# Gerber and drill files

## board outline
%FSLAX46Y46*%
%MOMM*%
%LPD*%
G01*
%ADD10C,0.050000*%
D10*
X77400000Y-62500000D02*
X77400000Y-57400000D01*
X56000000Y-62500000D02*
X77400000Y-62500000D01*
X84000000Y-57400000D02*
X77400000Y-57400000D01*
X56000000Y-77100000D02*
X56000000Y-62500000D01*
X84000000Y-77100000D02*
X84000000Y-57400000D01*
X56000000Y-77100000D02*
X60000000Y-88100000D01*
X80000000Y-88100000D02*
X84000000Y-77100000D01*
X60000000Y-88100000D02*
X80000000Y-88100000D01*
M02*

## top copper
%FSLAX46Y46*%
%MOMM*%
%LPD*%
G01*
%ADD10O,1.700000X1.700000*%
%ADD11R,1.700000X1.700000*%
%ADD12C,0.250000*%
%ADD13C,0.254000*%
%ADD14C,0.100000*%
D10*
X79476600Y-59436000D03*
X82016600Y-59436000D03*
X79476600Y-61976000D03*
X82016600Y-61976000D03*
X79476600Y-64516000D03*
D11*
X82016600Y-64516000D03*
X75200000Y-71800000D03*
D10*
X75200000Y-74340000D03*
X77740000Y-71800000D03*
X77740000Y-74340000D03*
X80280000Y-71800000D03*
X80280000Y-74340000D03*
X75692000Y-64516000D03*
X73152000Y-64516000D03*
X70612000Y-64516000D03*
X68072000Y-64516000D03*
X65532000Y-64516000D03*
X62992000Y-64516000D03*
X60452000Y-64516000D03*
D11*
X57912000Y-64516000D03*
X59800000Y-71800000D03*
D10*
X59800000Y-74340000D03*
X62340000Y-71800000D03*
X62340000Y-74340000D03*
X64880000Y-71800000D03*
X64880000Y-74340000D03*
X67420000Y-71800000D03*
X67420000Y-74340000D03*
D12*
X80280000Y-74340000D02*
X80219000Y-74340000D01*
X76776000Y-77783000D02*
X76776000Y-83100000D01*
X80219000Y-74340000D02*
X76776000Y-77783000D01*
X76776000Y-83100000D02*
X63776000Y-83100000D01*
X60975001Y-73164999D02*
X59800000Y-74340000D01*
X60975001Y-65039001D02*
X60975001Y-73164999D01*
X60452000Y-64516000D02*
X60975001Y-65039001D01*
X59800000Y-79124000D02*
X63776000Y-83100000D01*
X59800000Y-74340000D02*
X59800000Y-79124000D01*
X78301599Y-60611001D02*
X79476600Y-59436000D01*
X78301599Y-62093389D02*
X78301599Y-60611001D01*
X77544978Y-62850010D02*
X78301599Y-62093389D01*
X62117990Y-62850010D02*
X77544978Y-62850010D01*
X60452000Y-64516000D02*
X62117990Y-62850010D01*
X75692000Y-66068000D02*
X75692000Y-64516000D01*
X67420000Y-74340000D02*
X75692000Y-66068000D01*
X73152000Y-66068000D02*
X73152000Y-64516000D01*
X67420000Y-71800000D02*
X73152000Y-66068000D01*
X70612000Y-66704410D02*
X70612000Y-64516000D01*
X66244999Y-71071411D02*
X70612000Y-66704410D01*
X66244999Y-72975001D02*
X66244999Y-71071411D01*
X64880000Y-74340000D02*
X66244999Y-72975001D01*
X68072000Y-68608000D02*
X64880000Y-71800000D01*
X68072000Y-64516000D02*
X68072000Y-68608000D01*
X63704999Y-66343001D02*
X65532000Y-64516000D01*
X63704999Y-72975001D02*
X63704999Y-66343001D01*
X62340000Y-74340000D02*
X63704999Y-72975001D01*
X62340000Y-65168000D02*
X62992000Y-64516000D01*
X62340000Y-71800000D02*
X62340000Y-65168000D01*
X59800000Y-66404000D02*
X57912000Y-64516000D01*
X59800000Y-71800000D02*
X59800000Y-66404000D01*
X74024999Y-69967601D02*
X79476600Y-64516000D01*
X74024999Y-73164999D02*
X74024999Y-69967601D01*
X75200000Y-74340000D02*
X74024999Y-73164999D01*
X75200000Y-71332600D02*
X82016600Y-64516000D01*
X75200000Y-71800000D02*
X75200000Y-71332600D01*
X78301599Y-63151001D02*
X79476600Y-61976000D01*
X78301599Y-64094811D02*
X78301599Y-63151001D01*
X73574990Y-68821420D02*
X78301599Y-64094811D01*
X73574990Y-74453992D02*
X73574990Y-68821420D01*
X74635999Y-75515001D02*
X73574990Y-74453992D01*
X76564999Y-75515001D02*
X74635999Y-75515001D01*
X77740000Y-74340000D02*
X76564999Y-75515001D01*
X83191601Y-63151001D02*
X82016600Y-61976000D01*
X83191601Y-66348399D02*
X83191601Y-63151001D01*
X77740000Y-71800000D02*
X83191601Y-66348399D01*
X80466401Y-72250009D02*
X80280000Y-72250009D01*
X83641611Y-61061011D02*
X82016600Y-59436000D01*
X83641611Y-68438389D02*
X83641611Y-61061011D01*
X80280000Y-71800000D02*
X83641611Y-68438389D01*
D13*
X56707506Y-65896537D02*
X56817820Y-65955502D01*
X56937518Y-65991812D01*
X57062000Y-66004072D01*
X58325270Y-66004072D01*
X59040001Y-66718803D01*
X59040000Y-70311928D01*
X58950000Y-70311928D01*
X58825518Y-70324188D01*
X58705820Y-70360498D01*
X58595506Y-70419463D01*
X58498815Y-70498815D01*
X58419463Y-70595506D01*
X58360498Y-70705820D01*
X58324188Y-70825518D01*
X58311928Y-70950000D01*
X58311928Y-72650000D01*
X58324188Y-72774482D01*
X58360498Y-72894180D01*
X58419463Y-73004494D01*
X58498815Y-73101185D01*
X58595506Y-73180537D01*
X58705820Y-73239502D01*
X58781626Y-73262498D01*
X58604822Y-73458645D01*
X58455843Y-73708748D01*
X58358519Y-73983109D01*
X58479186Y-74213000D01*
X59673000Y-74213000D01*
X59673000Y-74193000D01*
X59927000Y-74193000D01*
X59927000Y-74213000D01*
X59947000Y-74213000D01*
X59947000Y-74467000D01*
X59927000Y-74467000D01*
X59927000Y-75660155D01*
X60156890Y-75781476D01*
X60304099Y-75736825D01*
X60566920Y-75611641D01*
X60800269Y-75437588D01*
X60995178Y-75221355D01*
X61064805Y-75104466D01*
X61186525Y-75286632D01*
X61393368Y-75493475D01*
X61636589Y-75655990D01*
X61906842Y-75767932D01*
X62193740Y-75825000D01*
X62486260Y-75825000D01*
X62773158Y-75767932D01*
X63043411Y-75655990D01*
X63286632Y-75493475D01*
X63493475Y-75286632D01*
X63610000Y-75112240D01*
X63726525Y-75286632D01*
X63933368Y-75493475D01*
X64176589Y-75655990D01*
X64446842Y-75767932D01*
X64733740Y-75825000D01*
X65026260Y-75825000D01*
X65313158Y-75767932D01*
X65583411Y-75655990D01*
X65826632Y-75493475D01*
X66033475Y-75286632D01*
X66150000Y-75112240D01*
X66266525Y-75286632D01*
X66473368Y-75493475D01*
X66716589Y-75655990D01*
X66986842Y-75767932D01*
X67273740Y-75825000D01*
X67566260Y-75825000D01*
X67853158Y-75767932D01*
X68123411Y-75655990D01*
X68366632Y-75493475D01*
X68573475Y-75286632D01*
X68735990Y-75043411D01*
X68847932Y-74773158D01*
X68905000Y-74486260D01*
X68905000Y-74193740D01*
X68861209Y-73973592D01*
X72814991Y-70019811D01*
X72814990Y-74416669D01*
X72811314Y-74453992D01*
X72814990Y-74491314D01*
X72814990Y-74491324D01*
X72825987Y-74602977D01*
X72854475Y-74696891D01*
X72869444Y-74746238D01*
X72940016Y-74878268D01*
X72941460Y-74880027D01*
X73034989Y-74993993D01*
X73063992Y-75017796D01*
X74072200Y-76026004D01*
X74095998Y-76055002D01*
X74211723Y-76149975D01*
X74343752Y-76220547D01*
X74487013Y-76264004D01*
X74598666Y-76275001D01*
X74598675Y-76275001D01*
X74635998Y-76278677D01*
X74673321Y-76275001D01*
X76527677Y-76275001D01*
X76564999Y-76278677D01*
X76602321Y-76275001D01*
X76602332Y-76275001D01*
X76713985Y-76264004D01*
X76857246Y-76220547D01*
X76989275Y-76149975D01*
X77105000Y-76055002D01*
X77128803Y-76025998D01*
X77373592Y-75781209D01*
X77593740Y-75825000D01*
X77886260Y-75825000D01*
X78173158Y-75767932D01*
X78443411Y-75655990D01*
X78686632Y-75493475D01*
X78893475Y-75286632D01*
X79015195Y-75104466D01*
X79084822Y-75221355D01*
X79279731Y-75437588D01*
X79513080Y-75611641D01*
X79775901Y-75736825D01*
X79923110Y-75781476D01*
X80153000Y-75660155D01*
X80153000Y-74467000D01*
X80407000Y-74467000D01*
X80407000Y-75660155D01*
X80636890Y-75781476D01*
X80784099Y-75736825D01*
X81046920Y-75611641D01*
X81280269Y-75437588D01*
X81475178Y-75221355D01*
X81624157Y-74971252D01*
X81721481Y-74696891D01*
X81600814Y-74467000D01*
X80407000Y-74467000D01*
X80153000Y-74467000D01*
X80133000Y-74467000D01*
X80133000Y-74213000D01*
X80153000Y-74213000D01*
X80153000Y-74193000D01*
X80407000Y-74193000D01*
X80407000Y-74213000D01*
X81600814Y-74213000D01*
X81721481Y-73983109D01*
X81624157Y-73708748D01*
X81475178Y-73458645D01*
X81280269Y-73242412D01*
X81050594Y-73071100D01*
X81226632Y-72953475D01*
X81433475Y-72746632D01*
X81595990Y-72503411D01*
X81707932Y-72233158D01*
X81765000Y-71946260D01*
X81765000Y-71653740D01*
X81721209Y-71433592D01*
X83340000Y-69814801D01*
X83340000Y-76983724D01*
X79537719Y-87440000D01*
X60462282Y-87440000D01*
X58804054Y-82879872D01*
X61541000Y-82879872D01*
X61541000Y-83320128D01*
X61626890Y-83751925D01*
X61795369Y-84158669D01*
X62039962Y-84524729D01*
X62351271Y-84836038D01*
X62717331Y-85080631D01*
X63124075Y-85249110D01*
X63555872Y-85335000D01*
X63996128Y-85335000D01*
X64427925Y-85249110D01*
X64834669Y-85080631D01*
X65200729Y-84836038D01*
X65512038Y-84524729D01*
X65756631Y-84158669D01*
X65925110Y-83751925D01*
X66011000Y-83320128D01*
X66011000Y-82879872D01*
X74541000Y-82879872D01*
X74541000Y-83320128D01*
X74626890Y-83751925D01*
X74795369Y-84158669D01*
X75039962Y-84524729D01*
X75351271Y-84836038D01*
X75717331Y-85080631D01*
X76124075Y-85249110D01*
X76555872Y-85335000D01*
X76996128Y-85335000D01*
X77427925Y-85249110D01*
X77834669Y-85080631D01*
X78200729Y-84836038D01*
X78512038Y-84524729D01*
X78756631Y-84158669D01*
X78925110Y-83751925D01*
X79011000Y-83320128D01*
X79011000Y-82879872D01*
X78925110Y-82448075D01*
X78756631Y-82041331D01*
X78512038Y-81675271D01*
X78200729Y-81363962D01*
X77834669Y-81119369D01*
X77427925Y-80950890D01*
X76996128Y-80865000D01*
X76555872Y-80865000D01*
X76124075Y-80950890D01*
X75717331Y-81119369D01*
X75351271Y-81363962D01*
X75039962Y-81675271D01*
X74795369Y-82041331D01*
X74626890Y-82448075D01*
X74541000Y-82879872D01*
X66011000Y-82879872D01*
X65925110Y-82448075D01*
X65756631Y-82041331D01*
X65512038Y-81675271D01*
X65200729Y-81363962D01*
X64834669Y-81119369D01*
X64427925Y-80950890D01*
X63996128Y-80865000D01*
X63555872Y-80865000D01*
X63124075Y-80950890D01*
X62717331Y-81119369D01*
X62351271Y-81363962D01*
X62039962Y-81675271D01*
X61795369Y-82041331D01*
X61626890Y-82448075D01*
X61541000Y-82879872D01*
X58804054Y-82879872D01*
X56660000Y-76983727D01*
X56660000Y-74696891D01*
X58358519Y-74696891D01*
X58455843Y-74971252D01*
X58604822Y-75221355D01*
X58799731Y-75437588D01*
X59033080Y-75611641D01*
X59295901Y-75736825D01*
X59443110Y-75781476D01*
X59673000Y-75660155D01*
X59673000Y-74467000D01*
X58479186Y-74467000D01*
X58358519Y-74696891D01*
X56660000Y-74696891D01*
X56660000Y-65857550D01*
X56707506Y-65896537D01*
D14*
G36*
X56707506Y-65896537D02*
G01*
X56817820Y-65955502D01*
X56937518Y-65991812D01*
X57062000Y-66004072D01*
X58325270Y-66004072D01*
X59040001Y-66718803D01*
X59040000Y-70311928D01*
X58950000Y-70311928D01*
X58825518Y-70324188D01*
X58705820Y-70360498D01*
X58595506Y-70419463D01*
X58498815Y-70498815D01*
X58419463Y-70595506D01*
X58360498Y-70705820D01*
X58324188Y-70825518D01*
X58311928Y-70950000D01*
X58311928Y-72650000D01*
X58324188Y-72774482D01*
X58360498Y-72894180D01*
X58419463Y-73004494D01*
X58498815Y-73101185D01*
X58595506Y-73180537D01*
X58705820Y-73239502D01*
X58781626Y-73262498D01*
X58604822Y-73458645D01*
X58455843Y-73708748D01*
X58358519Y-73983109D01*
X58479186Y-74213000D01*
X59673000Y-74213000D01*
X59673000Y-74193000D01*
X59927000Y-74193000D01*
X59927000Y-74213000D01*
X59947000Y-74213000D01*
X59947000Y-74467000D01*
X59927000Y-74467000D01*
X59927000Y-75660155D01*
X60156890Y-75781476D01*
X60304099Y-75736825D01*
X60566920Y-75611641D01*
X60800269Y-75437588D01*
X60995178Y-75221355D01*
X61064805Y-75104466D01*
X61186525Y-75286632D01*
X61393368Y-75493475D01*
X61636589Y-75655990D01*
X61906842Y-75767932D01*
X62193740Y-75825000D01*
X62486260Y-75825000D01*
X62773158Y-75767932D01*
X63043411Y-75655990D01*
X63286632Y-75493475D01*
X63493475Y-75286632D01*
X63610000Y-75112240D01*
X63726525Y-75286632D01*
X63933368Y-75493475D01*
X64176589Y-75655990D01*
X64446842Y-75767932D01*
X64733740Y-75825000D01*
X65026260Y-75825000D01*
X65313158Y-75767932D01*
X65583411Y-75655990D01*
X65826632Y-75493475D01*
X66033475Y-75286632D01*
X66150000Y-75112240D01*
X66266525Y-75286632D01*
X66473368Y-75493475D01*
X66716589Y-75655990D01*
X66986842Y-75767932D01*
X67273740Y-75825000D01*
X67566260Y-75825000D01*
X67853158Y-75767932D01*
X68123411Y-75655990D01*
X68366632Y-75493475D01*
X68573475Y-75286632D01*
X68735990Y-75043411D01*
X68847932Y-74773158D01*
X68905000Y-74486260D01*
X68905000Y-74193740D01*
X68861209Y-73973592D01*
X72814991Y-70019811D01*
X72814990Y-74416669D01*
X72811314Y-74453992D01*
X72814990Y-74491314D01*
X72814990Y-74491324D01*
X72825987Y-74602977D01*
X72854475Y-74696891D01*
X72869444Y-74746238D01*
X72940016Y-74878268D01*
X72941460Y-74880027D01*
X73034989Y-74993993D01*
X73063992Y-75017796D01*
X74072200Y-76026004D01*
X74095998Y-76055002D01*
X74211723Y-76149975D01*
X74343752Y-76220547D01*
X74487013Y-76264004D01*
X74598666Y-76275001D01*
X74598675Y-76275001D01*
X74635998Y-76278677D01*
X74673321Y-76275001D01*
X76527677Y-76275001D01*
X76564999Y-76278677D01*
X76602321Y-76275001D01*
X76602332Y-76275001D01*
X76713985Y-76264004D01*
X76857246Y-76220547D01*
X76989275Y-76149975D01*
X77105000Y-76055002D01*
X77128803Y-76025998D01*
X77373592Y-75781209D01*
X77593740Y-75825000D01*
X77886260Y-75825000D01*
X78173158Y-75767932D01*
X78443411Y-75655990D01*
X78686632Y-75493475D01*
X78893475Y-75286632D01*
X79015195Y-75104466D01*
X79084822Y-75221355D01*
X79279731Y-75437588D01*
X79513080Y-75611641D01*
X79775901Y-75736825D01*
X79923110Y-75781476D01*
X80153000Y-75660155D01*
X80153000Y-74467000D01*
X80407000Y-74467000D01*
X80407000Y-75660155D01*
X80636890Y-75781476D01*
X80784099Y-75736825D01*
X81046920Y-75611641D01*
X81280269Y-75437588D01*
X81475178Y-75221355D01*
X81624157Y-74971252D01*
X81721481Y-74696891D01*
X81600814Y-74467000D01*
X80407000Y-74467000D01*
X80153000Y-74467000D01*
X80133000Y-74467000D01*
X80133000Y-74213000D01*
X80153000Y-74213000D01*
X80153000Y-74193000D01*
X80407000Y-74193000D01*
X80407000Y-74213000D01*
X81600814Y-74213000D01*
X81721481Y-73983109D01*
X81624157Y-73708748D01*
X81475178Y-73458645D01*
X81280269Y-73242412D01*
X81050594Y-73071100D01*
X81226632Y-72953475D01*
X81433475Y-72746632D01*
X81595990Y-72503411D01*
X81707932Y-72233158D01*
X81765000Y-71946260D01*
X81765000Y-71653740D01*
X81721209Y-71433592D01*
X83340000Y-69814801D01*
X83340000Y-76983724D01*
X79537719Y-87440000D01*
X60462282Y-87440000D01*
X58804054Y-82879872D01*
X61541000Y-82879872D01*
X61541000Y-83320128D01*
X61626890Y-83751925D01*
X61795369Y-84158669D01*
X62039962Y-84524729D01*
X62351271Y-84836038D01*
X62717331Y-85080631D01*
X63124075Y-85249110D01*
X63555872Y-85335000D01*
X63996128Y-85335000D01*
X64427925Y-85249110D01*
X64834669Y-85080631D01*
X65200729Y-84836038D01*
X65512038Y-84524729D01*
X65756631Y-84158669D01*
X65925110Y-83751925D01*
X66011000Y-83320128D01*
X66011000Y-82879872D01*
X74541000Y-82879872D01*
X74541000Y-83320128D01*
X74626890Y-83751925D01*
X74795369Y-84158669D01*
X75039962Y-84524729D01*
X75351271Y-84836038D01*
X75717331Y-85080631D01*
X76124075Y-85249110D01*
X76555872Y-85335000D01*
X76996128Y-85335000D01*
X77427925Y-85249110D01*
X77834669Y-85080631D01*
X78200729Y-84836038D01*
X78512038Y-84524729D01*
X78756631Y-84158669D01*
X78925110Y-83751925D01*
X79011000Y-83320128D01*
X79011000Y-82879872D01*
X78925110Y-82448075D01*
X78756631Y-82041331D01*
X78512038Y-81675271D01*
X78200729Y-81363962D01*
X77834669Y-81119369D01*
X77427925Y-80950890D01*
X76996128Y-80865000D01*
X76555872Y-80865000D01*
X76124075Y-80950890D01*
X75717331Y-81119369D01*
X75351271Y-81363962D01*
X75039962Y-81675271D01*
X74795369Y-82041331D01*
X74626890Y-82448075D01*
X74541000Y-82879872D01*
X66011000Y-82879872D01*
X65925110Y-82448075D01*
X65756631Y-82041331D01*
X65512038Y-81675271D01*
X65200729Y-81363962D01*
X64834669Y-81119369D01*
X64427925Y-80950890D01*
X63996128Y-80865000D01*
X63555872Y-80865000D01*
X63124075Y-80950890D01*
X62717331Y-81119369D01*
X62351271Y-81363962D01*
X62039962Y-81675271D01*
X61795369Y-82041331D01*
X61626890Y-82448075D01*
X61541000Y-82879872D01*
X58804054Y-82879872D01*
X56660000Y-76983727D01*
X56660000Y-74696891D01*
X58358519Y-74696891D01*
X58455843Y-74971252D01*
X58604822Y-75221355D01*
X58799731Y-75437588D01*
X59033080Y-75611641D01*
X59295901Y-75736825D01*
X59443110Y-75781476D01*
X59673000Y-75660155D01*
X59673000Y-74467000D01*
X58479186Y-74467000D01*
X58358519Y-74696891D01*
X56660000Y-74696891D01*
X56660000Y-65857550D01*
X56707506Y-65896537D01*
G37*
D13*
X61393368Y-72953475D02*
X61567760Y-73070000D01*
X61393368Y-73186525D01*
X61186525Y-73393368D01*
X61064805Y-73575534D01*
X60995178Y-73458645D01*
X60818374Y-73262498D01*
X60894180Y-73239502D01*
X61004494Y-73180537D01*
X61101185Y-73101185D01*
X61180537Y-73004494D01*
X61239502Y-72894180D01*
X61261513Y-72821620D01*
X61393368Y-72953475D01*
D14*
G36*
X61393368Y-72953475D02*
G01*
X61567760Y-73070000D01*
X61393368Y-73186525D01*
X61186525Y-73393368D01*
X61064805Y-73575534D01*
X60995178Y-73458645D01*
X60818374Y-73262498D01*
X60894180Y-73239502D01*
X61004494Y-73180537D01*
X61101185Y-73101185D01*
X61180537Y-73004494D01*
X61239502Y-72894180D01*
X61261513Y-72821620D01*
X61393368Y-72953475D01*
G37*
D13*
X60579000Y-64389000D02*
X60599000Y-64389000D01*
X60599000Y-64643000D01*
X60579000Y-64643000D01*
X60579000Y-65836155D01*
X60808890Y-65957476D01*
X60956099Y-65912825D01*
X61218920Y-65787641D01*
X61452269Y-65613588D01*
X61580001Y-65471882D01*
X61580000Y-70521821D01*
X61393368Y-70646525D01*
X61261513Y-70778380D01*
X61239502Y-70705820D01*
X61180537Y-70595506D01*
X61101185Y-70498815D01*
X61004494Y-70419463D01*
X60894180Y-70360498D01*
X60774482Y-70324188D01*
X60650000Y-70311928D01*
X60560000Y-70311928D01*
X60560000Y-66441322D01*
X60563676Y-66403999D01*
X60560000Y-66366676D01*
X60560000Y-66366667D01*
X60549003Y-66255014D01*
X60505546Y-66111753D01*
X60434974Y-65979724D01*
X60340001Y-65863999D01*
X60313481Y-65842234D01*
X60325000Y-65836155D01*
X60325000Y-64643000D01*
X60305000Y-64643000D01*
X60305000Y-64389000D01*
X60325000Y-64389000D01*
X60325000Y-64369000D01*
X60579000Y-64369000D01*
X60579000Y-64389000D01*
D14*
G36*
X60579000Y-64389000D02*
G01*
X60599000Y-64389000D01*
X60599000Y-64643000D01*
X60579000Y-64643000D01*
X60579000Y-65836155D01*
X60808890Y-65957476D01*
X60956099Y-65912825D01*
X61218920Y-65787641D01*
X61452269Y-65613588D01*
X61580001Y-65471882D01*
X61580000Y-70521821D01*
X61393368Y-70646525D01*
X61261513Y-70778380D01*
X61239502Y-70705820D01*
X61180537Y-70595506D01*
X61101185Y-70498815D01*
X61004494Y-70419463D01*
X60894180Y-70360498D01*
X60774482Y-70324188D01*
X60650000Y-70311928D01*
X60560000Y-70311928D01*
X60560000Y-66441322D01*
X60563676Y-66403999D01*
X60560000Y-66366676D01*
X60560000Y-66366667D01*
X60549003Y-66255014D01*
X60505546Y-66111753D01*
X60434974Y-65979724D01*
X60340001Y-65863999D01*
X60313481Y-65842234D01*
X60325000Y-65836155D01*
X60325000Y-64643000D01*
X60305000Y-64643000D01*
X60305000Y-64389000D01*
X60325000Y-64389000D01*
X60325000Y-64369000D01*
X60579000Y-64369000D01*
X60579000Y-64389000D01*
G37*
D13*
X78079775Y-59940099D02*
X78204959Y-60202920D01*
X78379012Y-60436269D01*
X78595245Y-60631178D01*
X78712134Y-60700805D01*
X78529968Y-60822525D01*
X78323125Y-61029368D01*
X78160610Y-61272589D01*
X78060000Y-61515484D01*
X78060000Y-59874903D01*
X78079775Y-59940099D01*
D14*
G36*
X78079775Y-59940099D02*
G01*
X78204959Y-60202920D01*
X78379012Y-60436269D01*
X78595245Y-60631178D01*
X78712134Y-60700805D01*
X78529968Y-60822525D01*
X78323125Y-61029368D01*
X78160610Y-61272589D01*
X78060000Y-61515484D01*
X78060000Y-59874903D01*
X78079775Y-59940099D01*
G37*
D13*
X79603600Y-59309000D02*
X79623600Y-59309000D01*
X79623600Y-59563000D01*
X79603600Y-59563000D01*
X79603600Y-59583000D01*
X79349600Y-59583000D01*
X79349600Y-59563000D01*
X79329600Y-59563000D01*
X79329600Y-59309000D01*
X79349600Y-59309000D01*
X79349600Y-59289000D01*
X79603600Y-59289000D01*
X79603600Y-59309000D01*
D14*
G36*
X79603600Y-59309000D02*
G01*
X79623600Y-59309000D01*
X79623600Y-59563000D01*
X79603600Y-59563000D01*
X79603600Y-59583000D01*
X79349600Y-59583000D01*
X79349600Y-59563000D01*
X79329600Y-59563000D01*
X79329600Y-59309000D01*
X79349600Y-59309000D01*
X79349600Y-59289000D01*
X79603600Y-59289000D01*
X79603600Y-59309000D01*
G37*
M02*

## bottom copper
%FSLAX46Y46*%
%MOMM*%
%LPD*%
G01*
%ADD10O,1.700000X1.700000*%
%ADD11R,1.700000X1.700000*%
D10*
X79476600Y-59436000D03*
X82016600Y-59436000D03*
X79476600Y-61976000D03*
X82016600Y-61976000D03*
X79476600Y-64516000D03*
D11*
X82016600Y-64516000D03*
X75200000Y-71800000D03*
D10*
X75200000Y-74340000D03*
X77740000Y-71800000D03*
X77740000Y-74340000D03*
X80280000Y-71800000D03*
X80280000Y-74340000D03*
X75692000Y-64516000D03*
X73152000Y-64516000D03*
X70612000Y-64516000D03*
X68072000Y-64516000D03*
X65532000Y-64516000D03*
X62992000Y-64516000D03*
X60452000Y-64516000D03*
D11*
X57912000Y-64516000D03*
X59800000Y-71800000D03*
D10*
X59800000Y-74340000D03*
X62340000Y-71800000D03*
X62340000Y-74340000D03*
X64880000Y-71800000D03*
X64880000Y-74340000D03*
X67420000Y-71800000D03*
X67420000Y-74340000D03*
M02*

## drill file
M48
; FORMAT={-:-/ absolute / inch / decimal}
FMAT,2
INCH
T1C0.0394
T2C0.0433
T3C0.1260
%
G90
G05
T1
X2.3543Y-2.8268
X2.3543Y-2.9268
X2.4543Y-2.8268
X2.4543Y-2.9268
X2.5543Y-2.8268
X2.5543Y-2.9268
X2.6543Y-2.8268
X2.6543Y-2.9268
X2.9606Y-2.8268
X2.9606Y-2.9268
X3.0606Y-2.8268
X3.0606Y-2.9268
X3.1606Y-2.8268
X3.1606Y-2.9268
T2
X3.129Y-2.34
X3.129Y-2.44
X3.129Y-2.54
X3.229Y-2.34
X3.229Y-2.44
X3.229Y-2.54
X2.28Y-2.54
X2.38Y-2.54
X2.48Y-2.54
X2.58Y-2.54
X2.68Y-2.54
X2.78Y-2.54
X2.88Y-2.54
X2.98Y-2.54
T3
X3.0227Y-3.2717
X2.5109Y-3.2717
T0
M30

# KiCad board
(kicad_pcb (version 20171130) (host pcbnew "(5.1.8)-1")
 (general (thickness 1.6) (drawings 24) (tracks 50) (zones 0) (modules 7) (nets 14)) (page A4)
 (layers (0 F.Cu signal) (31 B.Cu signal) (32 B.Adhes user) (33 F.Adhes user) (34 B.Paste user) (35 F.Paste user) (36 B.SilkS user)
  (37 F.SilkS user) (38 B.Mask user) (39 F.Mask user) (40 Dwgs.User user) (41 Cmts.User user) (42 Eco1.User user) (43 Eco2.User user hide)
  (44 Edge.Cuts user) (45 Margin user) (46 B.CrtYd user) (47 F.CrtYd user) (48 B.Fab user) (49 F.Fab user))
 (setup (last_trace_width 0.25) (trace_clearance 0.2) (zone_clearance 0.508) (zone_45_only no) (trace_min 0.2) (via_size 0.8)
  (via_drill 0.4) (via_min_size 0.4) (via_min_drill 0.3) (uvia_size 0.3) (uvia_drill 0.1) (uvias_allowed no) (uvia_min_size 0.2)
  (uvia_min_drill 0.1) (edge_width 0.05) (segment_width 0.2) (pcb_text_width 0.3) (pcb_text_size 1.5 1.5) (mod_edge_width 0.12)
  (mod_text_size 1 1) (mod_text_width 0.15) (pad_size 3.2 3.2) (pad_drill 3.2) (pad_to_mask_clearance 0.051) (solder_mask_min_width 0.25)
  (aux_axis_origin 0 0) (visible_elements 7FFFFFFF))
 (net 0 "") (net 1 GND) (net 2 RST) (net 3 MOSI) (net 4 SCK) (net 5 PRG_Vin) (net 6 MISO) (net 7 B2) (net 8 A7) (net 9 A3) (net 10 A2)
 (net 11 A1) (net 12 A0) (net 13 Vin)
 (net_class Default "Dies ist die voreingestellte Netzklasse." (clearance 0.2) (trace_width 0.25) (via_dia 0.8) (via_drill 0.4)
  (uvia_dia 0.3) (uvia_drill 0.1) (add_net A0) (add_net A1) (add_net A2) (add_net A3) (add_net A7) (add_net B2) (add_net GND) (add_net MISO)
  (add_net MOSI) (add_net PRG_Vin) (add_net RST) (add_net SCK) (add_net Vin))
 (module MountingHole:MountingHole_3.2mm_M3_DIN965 (layer F.Cu) (at 63.6778 83.1342)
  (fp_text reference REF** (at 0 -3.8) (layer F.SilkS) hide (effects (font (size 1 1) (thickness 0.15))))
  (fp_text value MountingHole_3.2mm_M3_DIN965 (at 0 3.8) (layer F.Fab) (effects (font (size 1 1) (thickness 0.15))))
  (pad "" np_thru_hole circle (at 0.0982 -0.0342) (size 3.2 3.2) (drill 3.2) (layers *.Cu *.Mask)))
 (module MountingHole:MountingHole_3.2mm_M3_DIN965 (layer F.Cu) (at 76.776 83.1)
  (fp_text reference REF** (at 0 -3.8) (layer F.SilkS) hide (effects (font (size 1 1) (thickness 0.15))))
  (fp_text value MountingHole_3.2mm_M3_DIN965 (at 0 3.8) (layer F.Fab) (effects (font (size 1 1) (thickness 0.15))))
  (pad 1 np_thru_hole circle (at 0 0) (size 3.2 3.2) (drill 3.2) (layers *.Cu *.Mask)))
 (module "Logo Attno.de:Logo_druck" (layer F.Cu) (at 70.2056 82.042)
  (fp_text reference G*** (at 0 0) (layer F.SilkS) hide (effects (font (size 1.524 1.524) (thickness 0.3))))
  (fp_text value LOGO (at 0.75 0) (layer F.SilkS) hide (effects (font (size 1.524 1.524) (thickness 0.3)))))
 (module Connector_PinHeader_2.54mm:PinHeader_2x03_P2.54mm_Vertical (layer F.Cu) (at 82.0166 64.516 180)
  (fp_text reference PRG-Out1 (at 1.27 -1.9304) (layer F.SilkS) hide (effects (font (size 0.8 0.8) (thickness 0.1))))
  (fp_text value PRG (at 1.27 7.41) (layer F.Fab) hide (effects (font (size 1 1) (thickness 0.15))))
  (pad 6 thru_hole oval (at 2.54 5.08 180) (size 1.7 1.7) (drill 1.1) (layers *.Cu *.Mask) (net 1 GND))
  (pad 5 thru_hole oval (at 0 5.08 180) (size 1.7 1.7) (drill 1.1) (layers *.Cu *.Mask) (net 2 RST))
  (pad 4 thru_hole oval (at 2.54 2.54 180) (size 1.7 1.7) (drill 1.1) (layers *.Cu *.Mask) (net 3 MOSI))
  (pad 3 thru_hole oval (at 0 2.54 180) (size 1.7 1.7) (drill 1.1) (layers *.Cu *.Mask) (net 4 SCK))
  (pad 2 thru_hole oval (at 2.54 0 180) (size 1.7 1.7) (drill 1.1) (layers *.Cu *.Mask) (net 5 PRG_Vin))
  (pad 1 thru_hole rect (at 0 0 180) (size 1.7 1.7) (drill 1.1) (layers *.Cu *.Mask) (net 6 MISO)))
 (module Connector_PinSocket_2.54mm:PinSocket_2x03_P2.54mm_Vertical (layer F.Cu) (at 75.2 71.8 90)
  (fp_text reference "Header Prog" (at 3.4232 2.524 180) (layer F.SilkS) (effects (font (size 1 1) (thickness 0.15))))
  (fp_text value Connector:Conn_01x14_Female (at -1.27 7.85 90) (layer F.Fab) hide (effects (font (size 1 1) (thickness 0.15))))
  (pad 1 thru_hole rect (at 0 0 90) (size 1.7 1.7) (drill 1) (layers *.Cu *.Mask) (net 6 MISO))
  (pad 2 thru_hole oval (at -2.54 0 90) (size 1.7 1.7) (drill 1) (layers *.Cu *.Mask) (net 5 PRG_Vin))
  (pad 3 thru_hole oval (at 0 2.54 90) (size 1.7 1.7) (drill 1) (layers *.Cu *.Mask) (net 4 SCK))
  (pad 4 thru_hole oval (at -2.54 2.54 90) (size 1.7 1.7) (drill 1) (layers *.Cu *.Mask) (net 3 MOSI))
  (pad 5 thru_hole oval (at 0 5.08 90) (size 1.7 1.7) (drill 1) (layers *.Cu *.Mask) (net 2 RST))
  (pad 6 thru_hole oval (at -2.54 5.08 90) (size 1.7 1.7) (drill 1) (layers *.Cu *.Mask) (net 1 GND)))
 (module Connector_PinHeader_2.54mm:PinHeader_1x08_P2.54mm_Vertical (layer F.Cu) (at 57.912 64.516 90)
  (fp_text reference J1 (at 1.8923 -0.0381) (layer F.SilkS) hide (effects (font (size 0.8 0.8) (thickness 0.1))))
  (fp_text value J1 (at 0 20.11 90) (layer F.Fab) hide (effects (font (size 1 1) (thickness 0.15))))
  (pad 8 thru_hole oval (at 0 17.78 90) (size 1.7 1.7) (drill 1.1) (layers *.Cu *.Mask) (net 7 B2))
  (pad 7 thru_hole oval (at 0 15.24 90) (size 1.7 1.7) (drill 1.1) (layers *.Cu *.Mask) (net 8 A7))
  (pad 6 thru_hole oval (at 0 12.7 90) (size 1.7 1.7) (drill 1.1) (layers *.Cu *.Mask) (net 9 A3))
  (pad 5 thru_hole oval (at 0 10.16 90) (size 1.7 1.7) (drill 1.1) (layers *.Cu *.Mask) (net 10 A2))
  (pad 4 thru_hole oval (at 0 7.62 90) (size 1.7 1.7) (drill 1.1) (layers *.Cu *.Mask) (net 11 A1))
  (pad 3 thru_hole oval (at 0 5.08 90) (size 1.7 1.7) (drill 1.1) (layers *.Cu *.Mask) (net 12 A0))
  (pad 2 thru_hole oval (at 0 2.54 90) (size 1.7 1.7) (drill 1.1) (layers *.Cu *.Mask) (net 1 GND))
  (pad 1 thru_hole rect (at 0 0 90) (size 1.7 1.7) (drill 1.1) (layers *.Cu *.Mask) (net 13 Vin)))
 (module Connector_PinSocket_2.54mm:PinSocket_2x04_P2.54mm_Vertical (layer F.Cu) (at 59.8 71.8 90)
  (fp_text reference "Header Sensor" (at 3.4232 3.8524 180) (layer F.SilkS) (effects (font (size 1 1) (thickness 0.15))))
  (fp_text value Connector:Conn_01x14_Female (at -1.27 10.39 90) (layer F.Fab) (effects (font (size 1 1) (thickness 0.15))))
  (pad 1 thru_hole rect (at 0 0 90) (size 1.7 1.7) (drill 1) (layers *.Cu *.Mask) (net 13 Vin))
  (pad 2 thru_hole oval (at -2.54 0 90) (size 1.7 1.7) (drill 1) (layers *.Cu *.Mask) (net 1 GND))
  (pad 3 thru_hole oval (at 0 2.54 90) (size 1.7 1.7) (drill 1) (layers *.Cu *.Mask) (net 12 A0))
  (pad 4 thru_hole oval (at -2.54 2.54 90) (size 1.7 1.7) (drill 1) (layers *.Cu *.Mask) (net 11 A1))
  (pad 5 thru_hole oval (at 0 5.08 90) (size 1.7 1.7) (drill 1) (layers *.Cu *.Mask) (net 10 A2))
  (pad 6 thru_hole oval (at -2.54 5.08 90) (size 1.7 1.7) (drill 1) (layers *.Cu *.Mask) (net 9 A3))
  (pad 7 thru_hole oval (at 0 7.62 90) (size 1.7 1.7) (drill 1) (layers *.Cu *.Mask) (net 8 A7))
  (pad 8 thru_hole oval (at -2.54 7.62 90) (size 1.7 1.7) (drill 1) (layers *.Cu *.Mask) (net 7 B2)))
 (gr_line (start 77.4 62.5) (end 77.4 57.4) (layer Edge.Cuts) (width 0.05))
 (gr_line (start 56 62.5) (end 77.4 62.5) (layer Edge.Cuts) (width 0.05))
 (gr_line (start 84 57.4) (end 77.4 57.4) (layer Edge.Cuts) (width 0.05))
 (gr_line (start 56 77.1) (end 56 62.5) (layer Edge.Cuts) (width 0.05))
 (gr_line (start 84 77.1) (end 84 57.4) (layer Edge.Cuts) (width 0.05))
 (gr_line (start 56 77.1) (end 60 88.1) (layer Edge.Cuts) (width 0.05))
 (gr_line (start 80 88.1) (end 84 77.1) (layer Edge.Cuts) (width 0.05))
 (gr_line (start 60 88.1) (end 80 88.1) (layer Edge.Cuts) (width 0.05))
 (segment (start 80.28 74.34) (end 80.219 74.34) (width 0.25) (layer F.Cu) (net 1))
 (segment (start 76.776 77.783) (end 76.776 83.1) (width 0.25) (layer F.Cu) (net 1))
 (segment (start 80.219 74.34) (end 76.776 77.783) (width 0.25) (layer F.Cu) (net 1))
 (segment (start 76.776 83.1) (end 63.776 83.1) (width 0.25) (layer F.Cu) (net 1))
 (segment (start 60.975001 73.164999) (end 59.8 74.34) (width 0.25) (layer F.Cu) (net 1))
 (segment (start 60.975001 65.039001) (end 60.975001 73.164999) (width 0.25) (layer F.Cu) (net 1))
 (segment (start 60.452 64.516) (end 60.975001 65.039001) (width 0.25) (layer F.Cu) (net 1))
 (segment (start 59.8 79.124) (end 63.776 83.1) (width 0.25) (layer F.Cu) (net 1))
 (segment (start 59.8 74.34) (end 59.8 79.124) (width 0.25) (layer F.Cu) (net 1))
 (segment (start 78.301599 60.611001) (end 79.4766 59.436) (width 0.25) (layer F.Cu) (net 1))
 (segment (start 78.301599 62.093389) (end 78.301599 60.611001) (width 0.25) (layer F.Cu) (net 1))
 (segment (start 77.544978 62.85001) (end 78.301599 62.093389) (width 0.25) (layer F.Cu) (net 1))
 (segment (start 62.11799 62.85001) (end 77.544978 62.85001) (width 0.25) (layer F.Cu) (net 1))
 (segment (start 60.452 64.516) (end 62.11799 62.85001) (width 0.25) (layer F.Cu) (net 1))
 (segment (start 75.692 66.068) (end 75.692 64.516) (width 0.25) (layer F.Cu) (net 7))
 (segment (start 67.42 74.34) (end 75.692 66.068) (width 0.25) (layer F.Cu) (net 7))
 (segment (start 73.152 66.068) (end 73.152 64.516) (width 0.25) (layer F.Cu) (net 8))
 (segment (start 67.42 71.8) (end 73.152 66.068) (width 0.25) (layer F.Cu) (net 8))
 (segment (start 70.612 66.70441) (end 70.612 64.516) (width 0.25) (layer F.Cu) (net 9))
 (segment (start 66.244999 71.071411) (end 70.612 66.70441) (width 0.25) (layer F.Cu) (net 9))
 (segment (start 66.244999 72.975001) (end 66.244999 71.071411) (width 0.25) (layer F.Cu) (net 9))
 (segment (start 64.88 74.34) (end 66.244999 72.975001) (width 0.25) (layer F.Cu) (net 9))
 (segment (start 68.072 68.608) (end 64.88 71.8) (width 0.25) (layer F.Cu) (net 10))
 (segment (start 68.072 64.516) (end 68.072 68.608) (width 0.25) (layer F.Cu) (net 10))
 (segment (start 63.704999 66.343001) (end 65.532 64.516) (width 0.25) (layer F.Cu) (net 11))
 (segment (start 63.704999 72.975001) (end 63.704999 66.343001) (width 0.25) (layer F.Cu) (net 11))
 (segment (start 62.34 74.34) (end 63.704999 72.975001) (width 0.25) (layer F.Cu) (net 11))
 (segment (start 62.34 65.168) (end 62.992 64.516) (width 0.25) (layer F.Cu) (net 12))
 (segment (start 62.34 71.8) (end 62.34 65.168) (width 0.25) (layer F.Cu) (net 12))
 (segment (start 59.8 66.404) (end 57.912 64.516) (width 0.25) (layer F.Cu) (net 13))
 (segment (start 59.8 71.8) (end 59.8 66.404) (width 0.25) (layer F.Cu) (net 13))
 (segment (start 74.024999 69.967601) (end 79.4766 64.516) (width 0.25) (layer F.Cu) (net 5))
 (segment (start 74.024999 73.164999) (end 74.024999 69.967601) (width 0.25) (layer F.Cu) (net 5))
 (segment (start 75.2 74.34) (end 74.024999 73.164999) (width 0.25) (layer F.Cu) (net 5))
 (segment (start 75.2 71.3326) (end 82.0166 64.516) (width 0.25) (layer F.Cu) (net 6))
 (segment (start 75.2 71.8) (end 75.2 71.3326) (width 0.25) (layer F.Cu) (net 6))
 (segment (start 78.301599 63.151001) (end 79.4766 61.976) (width 0.25) (layer F.Cu) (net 3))
 (segment (start 78.301599 64.094811) (end 78.301599 63.151001) (width 0.25) (layer F.Cu) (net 3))
 (segment (start 73.57499 68.82142) (end 78.301599 64.094811) (width 0.25) (layer F.Cu) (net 3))
 (segment (start 73.57499 74.453992) (end 73.57499 68.82142) (width 0.25) (layer F.Cu) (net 3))
 (segment (start 74.635999 75.515001) (end 73.57499 74.453992) (width 0.25) (layer F.Cu) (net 3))
 (segment (start 76.564999 75.515001) (end 74.635999 75.515001) (width 0.25) (layer F.Cu) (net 3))
 (segment (start 77.74 74.34) (end 76.564999 75.515001) (width 0.25) (layer F.Cu) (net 3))
 (segment (start 83.191601 63.151001) (end 82.0166 61.976) (width 0.25) (layer F.Cu) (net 4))
 (segment (start 83.191601 66.348399) (end 83.191601 63.151001) (width 0.25) (layer F.Cu) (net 4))
 (segment (start 77.74 71.8) (end 83.191601 66.348399) (width 0.25) (layer F.Cu) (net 4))
 (segment (start 80.466401 72.250009) (end 80.28 72.250009) (width 0.25) (layer F.Cu) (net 2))
 (segment (start 83.641611 61.061011) (end 82.0166 59.436) (width 0.25) (layer F.Cu) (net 2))
 (segment (start 83.641611 68.438389) (end 83.641611 61.061011) (width 0.25) (layer F.Cu) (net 2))
 (segment (start 80.28 71.8) (end 83.641611 68.438389) (width 0.25) (layer F.Cu) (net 2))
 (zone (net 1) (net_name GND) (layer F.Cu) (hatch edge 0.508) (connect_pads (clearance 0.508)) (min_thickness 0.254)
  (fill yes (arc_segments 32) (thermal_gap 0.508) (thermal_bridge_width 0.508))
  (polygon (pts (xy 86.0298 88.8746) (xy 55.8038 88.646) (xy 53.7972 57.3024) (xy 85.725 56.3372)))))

